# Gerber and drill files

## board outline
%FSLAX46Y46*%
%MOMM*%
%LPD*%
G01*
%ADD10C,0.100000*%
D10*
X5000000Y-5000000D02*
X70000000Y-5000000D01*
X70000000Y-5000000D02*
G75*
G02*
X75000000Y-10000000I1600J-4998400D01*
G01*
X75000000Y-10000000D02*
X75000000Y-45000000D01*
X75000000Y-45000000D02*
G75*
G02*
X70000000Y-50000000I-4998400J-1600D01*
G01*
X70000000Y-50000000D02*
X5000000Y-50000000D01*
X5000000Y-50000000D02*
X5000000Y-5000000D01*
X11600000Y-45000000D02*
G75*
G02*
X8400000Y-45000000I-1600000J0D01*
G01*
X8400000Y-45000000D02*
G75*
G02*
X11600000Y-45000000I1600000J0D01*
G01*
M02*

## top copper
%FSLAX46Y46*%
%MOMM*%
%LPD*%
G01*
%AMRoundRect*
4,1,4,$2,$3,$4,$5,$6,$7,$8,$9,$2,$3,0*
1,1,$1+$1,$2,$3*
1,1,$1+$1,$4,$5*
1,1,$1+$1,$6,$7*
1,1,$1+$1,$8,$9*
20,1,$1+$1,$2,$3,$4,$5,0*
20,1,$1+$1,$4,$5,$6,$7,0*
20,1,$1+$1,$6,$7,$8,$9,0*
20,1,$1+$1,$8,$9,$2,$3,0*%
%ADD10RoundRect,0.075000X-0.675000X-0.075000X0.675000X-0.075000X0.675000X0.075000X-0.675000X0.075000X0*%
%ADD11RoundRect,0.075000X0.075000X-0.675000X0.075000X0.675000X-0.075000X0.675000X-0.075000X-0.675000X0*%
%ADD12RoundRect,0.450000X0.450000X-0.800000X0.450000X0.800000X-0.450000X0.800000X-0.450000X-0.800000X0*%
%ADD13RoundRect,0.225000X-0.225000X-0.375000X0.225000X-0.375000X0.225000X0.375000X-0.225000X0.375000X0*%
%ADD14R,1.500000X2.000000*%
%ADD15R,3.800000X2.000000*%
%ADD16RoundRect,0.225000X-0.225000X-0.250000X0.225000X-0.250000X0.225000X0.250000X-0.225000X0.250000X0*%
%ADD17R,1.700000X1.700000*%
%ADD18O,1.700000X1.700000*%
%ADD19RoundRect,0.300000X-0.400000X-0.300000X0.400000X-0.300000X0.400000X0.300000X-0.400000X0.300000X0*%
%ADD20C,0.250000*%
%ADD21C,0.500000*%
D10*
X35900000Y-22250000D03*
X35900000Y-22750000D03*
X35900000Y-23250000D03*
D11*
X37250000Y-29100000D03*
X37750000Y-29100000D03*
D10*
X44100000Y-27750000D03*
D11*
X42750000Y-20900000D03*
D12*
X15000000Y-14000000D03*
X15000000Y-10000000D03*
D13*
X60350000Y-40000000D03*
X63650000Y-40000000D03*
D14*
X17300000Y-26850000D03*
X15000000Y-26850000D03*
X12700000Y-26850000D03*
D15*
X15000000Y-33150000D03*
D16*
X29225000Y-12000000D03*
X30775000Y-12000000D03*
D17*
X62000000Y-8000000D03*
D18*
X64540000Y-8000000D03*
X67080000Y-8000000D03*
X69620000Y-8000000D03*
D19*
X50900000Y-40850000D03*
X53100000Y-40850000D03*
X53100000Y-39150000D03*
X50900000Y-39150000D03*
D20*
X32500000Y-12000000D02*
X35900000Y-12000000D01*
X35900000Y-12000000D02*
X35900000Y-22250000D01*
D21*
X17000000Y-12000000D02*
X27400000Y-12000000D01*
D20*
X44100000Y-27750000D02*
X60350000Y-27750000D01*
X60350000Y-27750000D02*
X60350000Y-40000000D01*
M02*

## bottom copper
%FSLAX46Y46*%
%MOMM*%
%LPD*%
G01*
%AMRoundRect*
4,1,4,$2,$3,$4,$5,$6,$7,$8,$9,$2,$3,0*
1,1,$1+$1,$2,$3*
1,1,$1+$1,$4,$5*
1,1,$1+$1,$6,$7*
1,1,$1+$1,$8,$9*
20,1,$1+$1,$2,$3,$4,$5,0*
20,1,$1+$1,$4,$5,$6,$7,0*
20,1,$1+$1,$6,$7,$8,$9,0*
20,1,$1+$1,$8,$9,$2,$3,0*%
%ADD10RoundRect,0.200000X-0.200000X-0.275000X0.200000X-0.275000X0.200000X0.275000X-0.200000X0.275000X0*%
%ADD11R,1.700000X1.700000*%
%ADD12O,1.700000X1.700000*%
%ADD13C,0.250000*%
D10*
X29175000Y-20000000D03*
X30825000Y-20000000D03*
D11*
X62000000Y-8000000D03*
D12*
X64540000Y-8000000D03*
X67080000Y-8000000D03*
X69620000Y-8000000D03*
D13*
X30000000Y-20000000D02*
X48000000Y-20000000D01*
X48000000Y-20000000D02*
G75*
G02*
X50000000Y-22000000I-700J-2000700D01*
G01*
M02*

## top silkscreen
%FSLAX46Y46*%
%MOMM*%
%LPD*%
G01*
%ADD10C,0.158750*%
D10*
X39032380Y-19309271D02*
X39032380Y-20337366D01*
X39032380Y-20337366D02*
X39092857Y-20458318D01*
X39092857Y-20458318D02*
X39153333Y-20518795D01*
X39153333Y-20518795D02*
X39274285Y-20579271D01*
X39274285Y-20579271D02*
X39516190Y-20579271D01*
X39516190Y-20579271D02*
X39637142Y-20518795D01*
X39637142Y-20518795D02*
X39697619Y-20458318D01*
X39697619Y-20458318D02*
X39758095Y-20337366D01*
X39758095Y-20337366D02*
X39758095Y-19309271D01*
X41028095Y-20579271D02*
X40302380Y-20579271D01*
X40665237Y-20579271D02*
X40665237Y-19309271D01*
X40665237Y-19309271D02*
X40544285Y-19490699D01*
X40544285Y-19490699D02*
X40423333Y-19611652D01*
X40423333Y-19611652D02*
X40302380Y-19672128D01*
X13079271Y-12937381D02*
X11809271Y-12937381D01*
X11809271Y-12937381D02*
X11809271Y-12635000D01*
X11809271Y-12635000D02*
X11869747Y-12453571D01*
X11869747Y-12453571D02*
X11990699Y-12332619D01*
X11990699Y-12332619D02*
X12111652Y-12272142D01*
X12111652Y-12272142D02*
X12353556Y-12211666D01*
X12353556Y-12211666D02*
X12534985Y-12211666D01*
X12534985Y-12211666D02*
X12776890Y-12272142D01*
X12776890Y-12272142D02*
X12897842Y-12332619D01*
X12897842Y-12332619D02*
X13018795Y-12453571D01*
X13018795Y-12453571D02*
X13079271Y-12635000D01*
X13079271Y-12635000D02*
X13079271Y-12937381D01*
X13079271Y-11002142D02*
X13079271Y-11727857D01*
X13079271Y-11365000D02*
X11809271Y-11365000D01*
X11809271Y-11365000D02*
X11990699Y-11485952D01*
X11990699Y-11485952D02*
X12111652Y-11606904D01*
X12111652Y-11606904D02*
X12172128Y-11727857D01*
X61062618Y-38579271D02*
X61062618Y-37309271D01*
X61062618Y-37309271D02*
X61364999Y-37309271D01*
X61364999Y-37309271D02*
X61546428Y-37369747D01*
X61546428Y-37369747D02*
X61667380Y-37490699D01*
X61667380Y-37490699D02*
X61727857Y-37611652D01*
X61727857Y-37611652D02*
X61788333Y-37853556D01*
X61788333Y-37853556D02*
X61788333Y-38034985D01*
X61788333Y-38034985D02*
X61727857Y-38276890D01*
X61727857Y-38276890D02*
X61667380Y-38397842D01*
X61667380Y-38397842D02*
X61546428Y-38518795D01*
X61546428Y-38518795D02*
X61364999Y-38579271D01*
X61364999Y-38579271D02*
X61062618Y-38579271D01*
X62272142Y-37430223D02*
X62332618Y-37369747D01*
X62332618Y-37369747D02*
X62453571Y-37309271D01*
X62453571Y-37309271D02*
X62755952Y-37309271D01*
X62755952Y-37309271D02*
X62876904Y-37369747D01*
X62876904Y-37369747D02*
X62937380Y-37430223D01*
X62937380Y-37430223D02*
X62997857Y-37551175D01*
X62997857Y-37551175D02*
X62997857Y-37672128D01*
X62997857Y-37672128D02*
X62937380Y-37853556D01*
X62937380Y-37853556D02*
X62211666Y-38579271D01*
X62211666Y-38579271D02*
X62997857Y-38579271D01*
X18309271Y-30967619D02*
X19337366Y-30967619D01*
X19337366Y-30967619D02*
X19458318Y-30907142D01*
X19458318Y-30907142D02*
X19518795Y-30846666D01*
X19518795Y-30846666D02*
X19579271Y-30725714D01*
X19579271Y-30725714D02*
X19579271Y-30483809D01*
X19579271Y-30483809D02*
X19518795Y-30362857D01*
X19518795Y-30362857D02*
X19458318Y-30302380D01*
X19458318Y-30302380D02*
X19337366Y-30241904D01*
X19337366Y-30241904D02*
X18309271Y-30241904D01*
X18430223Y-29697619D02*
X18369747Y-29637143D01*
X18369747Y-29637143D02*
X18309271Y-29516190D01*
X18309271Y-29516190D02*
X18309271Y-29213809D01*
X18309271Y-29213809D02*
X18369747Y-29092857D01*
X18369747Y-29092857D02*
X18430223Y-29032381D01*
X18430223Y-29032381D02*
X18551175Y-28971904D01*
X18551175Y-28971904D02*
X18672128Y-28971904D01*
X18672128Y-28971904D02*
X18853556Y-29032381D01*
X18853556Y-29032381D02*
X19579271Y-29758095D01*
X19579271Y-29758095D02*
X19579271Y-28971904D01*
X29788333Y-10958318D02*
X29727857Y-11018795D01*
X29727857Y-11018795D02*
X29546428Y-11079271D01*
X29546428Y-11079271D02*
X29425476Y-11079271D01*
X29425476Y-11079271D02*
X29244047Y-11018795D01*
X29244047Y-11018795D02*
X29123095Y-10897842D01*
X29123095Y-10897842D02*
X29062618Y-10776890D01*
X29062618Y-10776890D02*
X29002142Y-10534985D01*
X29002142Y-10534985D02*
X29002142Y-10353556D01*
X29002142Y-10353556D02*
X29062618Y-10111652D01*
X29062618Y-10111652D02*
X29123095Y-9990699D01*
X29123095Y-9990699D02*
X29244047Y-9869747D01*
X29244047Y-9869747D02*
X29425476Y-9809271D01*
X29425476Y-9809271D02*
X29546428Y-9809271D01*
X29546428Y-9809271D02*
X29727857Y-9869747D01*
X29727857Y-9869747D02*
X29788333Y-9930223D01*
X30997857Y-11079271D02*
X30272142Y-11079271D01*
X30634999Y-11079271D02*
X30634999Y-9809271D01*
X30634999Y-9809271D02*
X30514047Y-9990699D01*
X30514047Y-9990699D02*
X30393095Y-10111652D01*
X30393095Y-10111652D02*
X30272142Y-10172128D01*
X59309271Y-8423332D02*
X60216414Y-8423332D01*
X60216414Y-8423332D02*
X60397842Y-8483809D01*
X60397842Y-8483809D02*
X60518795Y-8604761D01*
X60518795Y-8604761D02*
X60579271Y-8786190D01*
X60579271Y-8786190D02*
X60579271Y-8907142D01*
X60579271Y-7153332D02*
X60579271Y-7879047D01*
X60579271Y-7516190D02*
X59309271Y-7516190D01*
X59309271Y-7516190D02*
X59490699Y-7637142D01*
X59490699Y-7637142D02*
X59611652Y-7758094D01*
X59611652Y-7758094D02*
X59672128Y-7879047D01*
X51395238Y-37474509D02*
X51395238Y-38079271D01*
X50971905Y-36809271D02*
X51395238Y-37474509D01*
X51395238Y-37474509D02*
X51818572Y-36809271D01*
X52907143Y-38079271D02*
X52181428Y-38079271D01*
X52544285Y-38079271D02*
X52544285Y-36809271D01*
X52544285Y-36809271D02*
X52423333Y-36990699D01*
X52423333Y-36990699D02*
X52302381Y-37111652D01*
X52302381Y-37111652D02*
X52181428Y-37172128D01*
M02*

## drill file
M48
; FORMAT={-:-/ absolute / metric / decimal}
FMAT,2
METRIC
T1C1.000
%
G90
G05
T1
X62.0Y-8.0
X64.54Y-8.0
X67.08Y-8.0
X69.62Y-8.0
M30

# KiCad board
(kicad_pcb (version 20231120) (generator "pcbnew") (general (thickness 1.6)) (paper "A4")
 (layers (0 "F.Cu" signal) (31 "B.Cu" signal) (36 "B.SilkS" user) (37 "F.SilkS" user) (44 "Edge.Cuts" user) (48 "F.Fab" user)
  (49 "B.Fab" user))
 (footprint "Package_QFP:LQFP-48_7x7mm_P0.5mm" (layer "F.Cu") (at 40 25) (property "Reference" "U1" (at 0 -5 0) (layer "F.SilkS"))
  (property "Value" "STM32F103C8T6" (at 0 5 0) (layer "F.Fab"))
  (pad "1" smd roundrect (at -4.1 -2.75) (size 1.5 0.3) (layers "F.Cu" "F.Paste" "F.Mask"))
  (pad "2" smd roundrect (at -4.1 -2.25) (size 1.5 0.3) (layers "F.Cu" "F.Paste" "F.Mask"))
  (pad "3" smd roundrect (at -4.1 -1.75) (size 1.5 0.3) (layers "F.Cu" "F.Paste" "F.Mask"))
  (pad "13" smd roundrect (at -2.75 4.1 90) (size 1.5 0.3) (layers "F.Cu" "F.Paste" "F.Mask"))
  (pad "14" smd roundrect (at -2.25 4.1 90) (size 1.5 0.3) (layers "F.Cu" "F.Paste" "F.Mask"))
  (pad "25" smd roundrect (at 4.1 2.75) (size 1.5 0.3) (layers "F.Cu" "F.Paste" "F.Mask"))
  (pad "37" smd roundrect (at 2.75 -4.1 90) (size 1.5 0.3) (layers "F.Cu" "F.Paste" "F.Mask")))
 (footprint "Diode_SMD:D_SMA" (layer "F.Cu") (at 15 12 90) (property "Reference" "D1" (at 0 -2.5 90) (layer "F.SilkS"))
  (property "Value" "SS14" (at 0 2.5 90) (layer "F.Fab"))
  (pad "1" smd roundrect (at -2 0 90) (size 2.5 1.8) (layers "F.Cu" "F.Paste" "F.Mask"))
  (pad "2" smd roundrect (at 2 0 90) (size 2.5 1.8) (layers "F.Cu" "F.Paste" "F.Mask")))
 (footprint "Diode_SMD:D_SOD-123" (layer "F.Cu") (at 62 40) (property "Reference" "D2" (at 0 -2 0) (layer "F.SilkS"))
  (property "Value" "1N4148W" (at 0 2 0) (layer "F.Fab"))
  (pad "1" smd roundrect (at -1.65 0) (size 0.9 1.2) (layers "F.Cu" "F.Paste" "F.Mask"))
  (pad "2" smd roundrect (at 1.65 0) (size 0.9 1.2) (layers "F.Cu" "F.Paste" "F.Mask")))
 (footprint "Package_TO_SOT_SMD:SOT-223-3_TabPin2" (layer "F.Cu") (at 15 30 270) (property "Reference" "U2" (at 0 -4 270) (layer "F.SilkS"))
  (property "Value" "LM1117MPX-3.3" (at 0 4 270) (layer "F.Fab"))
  (pad "1" smd rect (at -3.15 -2.3 270) (size 2 1.5) (layers "F.Cu" "F.Paste" "F.Mask"))
  (pad "2" smd rect (at -3.15 0 270) (size 2 1.5) (layers "F.Cu" "F.Paste" "F.Mask"))
  (pad "3" smd rect (at -3.15 2.3 270) (size 2 1.5) (layers "F.Cu" "F.Paste" "F.Mask"))
  (pad "4" smd rect (at 3.15 0 270) (size 2 3.8) (layers "F.Cu" "F.Paste" "F.Mask")))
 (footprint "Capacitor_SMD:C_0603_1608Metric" (layer "F.Cu") (at 30 12) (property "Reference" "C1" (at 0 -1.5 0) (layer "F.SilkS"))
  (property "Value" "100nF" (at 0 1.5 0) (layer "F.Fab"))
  (pad "1" smd roundrect (at -0.775 0) (size 0.9 0.95) (layers "F.Cu" "F.Paste" "F.Mask"))
  (pad "2" smd roundrect (at 0.775 0) (size 0.9 0.95) (layers "F.Cu" "F.Paste" "F.Mask")))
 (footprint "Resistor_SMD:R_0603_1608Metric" (layer "B.Cu") (at 30 20) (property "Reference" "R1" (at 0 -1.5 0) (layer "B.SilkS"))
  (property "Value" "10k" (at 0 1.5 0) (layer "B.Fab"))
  (pad "1" smd roundrect (at -0.825 0) (size 0.8 0.95) (layers "B.Cu" "B.Paste" "B.Mask"))
  (pad "2" smd roundrect (at 0.825 0) (size 0.8 0.95) (layers "B.Cu" "B.Paste" "B.Mask")))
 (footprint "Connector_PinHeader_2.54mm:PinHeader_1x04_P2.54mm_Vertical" (layer "F.Cu") (at 62 8 90)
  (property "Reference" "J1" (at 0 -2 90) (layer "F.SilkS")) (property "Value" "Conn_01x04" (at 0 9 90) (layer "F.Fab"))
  (pad "1" thru_hole rect (at 0 0 90) (size 1.7 1.7) (drill 1) (layers "*.Cu" "*.Mask"))
  (pad "2" thru_hole oval (at 0 2.54 90) (size 1.7 1.7) (drill 1) (layers "*.Cu" "*.Mask"))
  (pad "3" thru_hole oval (at 0 5.08 90) (size 1.7 1.7) (drill 1) (layers "*.Cu" "*.Mask"))
  (pad "4" thru_hole oval (at 0 7.62 90) (size 1.7 1.7) (drill 1) (layers "*.Cu" "*.Mask")))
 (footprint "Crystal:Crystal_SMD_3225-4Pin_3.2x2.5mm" (layer "F.Cu") (at 52 40) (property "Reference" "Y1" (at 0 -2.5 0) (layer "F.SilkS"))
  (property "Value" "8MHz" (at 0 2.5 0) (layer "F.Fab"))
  (pad "1" smd roundrect (at -1.1 0.85) (size 1.4 1.2) (layers "F.Cu" "F.Paste" "F.Mask"))
  (pad "2" smd roundrect (at 1.1 0.85) (size 1.4 1.2) (layers "F.Cu" "F.Paste" "F.Mask"))
  (pad "3" smd roundrect (at 1.1 -0.85) (size 1.4 1.2) (layers "F.Cu" "F.Paste" "F.Mask"))
  (pad "4" smd roundrect (at -1.1 -0.85) (size 1.4 1.2) (layers "F.Cu" "F.Paste" "F.Mask")))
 (gr_line (start 5 5) (end 70 5) (layer "Edge.Cuts") (width 0.1))
 (gr_arc (start 70 5) (mid 73.536 6.464) (end 75 10) (layer "Edge.Cuts") (width 0.1))
 (gr_line (start 75 10) (end 75 45) (layer "Edge.Cuts") (width 0.1))
 (gr_arc (start 75 45) (mid 73.536 48.536) (end 70 50) (layer "Edge.Cuts") (width 0.1))
 (gr_line (start 70 50) (end 5 50) (layer "Edge.Cuts") (width 0.1))
 (gr_line (start 5 50) (end 5 5) (layer "Edge.Cuts") (width 0.1))
 (gr_circle (center 10 45) (end 11.6 45) (layer "Edge.Cuts") (width 0.1))
 (segment (start 32.5 12) (end 35.9 12) (width 0.25) (layer "F.Cu") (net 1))
 (segment (start 35.9 12) (end 35.9 22.25) (width 0.25) (layer "F.Cu") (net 1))
 (segment (start 17 12) (end 27.4 12) (width 0.5) (layer "F.Cu") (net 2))
 (segment (start 44.1 27.75) (end 60.35 27.75) (width 0.25) (layer "F.Cu") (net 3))
 (segment (start 60.35 27.75) (end 60.35 40) (width 0.25) (layer "F.Cu") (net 3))
 (segment (start 30 20) (end 48 20) (width 0.25) (layer "B.Cu") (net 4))
 (arc (start 48 20) (mid 49.414 20.586) (end 50 22) (width 0.25) (layer "B.Cu") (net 4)))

